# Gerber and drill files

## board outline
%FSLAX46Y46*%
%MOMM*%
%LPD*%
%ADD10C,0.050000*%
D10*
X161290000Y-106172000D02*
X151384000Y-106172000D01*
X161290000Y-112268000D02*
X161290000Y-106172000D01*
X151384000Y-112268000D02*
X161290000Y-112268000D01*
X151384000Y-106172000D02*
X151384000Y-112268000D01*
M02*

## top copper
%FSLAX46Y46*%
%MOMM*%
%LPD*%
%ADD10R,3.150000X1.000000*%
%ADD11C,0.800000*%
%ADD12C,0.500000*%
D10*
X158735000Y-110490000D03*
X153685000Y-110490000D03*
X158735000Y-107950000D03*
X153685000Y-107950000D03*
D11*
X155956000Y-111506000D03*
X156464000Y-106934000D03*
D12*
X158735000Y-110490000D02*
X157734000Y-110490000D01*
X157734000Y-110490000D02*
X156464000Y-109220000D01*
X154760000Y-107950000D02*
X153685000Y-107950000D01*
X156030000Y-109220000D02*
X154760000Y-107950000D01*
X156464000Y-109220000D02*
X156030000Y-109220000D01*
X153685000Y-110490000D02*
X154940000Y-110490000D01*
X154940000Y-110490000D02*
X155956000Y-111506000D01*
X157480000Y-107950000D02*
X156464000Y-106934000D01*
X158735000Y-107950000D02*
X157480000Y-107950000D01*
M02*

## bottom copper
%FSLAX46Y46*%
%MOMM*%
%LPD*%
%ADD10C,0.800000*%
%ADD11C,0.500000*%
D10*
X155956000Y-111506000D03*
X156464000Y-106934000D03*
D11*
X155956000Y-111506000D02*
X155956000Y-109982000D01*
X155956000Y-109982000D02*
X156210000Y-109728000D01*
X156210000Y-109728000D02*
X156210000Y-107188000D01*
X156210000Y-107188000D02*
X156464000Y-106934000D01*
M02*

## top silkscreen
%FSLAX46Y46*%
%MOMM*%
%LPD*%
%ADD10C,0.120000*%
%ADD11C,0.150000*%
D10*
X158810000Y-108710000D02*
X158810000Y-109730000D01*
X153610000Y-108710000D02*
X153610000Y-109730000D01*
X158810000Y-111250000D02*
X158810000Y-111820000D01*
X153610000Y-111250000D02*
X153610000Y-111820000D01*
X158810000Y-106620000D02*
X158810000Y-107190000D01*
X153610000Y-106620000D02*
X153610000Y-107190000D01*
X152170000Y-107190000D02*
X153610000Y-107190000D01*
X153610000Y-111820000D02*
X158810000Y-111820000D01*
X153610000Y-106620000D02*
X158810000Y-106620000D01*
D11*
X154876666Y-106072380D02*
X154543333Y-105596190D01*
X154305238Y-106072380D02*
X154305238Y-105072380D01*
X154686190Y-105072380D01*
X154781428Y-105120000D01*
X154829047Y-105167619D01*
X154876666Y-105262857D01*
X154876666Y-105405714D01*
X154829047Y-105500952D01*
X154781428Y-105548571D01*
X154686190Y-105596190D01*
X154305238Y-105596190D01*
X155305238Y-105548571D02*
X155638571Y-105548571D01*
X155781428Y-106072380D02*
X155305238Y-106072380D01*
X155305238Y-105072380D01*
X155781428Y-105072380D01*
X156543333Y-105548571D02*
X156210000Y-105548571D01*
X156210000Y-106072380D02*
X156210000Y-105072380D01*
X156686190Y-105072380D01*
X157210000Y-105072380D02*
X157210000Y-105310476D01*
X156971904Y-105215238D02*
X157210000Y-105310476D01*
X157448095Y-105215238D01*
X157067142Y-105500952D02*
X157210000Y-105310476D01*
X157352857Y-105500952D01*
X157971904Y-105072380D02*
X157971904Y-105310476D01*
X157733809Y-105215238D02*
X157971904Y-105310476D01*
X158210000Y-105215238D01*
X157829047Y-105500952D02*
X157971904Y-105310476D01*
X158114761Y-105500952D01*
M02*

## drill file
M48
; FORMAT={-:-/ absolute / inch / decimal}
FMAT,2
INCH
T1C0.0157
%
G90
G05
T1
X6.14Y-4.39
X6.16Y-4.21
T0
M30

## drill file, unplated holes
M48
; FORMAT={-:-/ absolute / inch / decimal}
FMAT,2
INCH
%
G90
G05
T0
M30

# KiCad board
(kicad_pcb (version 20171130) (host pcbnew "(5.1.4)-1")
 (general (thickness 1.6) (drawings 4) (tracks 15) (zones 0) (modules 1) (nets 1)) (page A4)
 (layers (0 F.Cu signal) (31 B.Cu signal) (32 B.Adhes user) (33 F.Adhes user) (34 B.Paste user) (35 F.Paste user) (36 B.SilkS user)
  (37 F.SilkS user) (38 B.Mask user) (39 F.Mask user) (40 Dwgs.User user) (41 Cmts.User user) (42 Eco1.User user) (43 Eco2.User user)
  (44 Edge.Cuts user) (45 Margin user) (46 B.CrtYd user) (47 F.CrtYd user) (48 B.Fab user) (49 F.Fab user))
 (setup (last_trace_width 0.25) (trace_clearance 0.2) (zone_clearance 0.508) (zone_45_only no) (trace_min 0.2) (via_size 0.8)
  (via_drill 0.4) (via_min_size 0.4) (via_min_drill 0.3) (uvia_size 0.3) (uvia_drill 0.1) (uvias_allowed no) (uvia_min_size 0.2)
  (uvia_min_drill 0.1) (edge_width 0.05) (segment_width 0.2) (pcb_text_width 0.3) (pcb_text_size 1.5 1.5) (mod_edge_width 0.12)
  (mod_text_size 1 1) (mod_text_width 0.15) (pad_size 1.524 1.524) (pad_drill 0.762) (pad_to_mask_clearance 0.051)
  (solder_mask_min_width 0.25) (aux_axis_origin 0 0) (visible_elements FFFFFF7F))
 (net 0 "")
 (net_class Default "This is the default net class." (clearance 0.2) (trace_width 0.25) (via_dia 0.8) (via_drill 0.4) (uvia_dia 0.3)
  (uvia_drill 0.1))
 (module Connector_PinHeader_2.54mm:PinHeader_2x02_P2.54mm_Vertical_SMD (layer F.Cu) (at 156.21 109.22)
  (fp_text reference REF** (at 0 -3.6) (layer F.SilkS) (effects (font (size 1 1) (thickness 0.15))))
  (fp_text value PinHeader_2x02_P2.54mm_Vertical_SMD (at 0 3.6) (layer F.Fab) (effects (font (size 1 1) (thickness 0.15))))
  (fp_line (start 2.6 -0.51) (end 2.6 0.51) (layer F.SilkS) (width 0.12))
  (fp_line (start -2.6 -0.51) (end -2.6 0.51) (layer F.SilkS) (width 0.12))
  (fp_line (start 2.6 2.03) (end 2.6 2.6) (layer F.SilkS) (width 0.12))
  (fp_line (start -2.6 2.03) (end -2.6 2.6) (layer F.SilkS) (width 0.12))
  (fp_line (start 2.6 -2.6) (end 2.6 -2.03) (layer F.SilkS) (width 0.12))
  (fp_line (start -2.6 -2.6) (end -2.6 -2.03) (layer F.SilkS) (width 0.12))
  (fp_line (start -4.04 -2.03) (end -2.6 -2.03) (layer F.SilkS) (width 0.12))
  (fp_line (start -2.6 2.6) (end 2.6 2.6) (layer F.SilkS) (width 0.12))
  (fp_line (start -2.6 -2.6) (end 2.6 -2.6) (layer F.SilkS) (width 0.12))
  (pad 4 smd rect (at 2.525 1.27) (size 3.15 1) (layers F.Cu F.Paste F.Mask))
  (pad 3 smd rect (at -2.525 1.27) (size 3.15 1) (layers F.Cu F.Paste F.Mask))
  (pad 2 smd rect (at 2.525 -1.27) (size 3.15 1) (layers F.Cu F.Paste F.Mask))
  (pad 1 smd rect (at -2.525 -1.27) (size 3.15 1) (layers F.Cu F.Paste F.Mask)))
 (gr_line (start 161.29 106.172) (end 151.384 106.172) (layer Edge.Cuts) (width 0.05))
 (gr_line (start 161.29 112.268) (end 161.29 106.172) (layer Edge.Cuts) (width 0.05))
 (gr_line (start 151.384 112.268) (end 161.29 112.268) (layer Edge.Cuts) (width 0.05))
 (gr_line (start 151.384 106.172) (end 151.384 112.268) (layer Edge.Cuts) (width 0.05))
 (segment (start 158.735 110.49) (end 157.734 110.49) (width 0.5) (layer F.Cu) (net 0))
 (segment (start 157.734 110.49) (end 156.464 109.22) (width 0.5) (layer F.Cu) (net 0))
 (segment (start 154.76 107.95) (end 153.685 107.95) (width 0.5) (layer F.Cu) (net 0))
 (segment (start 156.03 109.22) (end 154.76 107.95) (width 0.5) (layer F.Cu) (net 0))
 (segment (start 156.464 109.22) (end 156.03 109.22) (width 0.5) (layer F.Cu) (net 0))
 (via (at 155.956 111.506) (size 0.8) (drill 0.4) (layers F.Cu B.Cu) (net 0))
 (segment (start 153.685 110.49) (end 154.94 110.49) (width 0.5) (layer F.Cu) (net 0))
 (segment (start 154.94 110.49) (end 155.956 111.506) (width 0.5) (layer F.Cu) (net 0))
 (segment (start 155.956 111.506) (end 155.956 109.982) (width 0.5) (layer B.Cu) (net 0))
 (segment (start 155.956 109.982) (end 156.21 109.728) (width 0.5) (layer B.Cu) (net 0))
 (via (at 156.464 106.934) (size 0.8) (drill 0.4) (layers F.Cu B.Cu) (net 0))
 (segment (start 156.21 109.728) (end 156.21 107.188) (width 0.5) (layer B.Cu) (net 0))
 (segment (start 156.21 107.188) (end 156.464 106.934) (width 0.5) (layer B.Cu) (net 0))
 (segment (start 157.48 107.95) (end 156.464 106.934) (width 0.5) (layer F.Cu) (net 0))
 (segment (start 158.735 107.95) (end 157.48 107.95) (width 0.5) (layer F.Cu) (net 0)))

